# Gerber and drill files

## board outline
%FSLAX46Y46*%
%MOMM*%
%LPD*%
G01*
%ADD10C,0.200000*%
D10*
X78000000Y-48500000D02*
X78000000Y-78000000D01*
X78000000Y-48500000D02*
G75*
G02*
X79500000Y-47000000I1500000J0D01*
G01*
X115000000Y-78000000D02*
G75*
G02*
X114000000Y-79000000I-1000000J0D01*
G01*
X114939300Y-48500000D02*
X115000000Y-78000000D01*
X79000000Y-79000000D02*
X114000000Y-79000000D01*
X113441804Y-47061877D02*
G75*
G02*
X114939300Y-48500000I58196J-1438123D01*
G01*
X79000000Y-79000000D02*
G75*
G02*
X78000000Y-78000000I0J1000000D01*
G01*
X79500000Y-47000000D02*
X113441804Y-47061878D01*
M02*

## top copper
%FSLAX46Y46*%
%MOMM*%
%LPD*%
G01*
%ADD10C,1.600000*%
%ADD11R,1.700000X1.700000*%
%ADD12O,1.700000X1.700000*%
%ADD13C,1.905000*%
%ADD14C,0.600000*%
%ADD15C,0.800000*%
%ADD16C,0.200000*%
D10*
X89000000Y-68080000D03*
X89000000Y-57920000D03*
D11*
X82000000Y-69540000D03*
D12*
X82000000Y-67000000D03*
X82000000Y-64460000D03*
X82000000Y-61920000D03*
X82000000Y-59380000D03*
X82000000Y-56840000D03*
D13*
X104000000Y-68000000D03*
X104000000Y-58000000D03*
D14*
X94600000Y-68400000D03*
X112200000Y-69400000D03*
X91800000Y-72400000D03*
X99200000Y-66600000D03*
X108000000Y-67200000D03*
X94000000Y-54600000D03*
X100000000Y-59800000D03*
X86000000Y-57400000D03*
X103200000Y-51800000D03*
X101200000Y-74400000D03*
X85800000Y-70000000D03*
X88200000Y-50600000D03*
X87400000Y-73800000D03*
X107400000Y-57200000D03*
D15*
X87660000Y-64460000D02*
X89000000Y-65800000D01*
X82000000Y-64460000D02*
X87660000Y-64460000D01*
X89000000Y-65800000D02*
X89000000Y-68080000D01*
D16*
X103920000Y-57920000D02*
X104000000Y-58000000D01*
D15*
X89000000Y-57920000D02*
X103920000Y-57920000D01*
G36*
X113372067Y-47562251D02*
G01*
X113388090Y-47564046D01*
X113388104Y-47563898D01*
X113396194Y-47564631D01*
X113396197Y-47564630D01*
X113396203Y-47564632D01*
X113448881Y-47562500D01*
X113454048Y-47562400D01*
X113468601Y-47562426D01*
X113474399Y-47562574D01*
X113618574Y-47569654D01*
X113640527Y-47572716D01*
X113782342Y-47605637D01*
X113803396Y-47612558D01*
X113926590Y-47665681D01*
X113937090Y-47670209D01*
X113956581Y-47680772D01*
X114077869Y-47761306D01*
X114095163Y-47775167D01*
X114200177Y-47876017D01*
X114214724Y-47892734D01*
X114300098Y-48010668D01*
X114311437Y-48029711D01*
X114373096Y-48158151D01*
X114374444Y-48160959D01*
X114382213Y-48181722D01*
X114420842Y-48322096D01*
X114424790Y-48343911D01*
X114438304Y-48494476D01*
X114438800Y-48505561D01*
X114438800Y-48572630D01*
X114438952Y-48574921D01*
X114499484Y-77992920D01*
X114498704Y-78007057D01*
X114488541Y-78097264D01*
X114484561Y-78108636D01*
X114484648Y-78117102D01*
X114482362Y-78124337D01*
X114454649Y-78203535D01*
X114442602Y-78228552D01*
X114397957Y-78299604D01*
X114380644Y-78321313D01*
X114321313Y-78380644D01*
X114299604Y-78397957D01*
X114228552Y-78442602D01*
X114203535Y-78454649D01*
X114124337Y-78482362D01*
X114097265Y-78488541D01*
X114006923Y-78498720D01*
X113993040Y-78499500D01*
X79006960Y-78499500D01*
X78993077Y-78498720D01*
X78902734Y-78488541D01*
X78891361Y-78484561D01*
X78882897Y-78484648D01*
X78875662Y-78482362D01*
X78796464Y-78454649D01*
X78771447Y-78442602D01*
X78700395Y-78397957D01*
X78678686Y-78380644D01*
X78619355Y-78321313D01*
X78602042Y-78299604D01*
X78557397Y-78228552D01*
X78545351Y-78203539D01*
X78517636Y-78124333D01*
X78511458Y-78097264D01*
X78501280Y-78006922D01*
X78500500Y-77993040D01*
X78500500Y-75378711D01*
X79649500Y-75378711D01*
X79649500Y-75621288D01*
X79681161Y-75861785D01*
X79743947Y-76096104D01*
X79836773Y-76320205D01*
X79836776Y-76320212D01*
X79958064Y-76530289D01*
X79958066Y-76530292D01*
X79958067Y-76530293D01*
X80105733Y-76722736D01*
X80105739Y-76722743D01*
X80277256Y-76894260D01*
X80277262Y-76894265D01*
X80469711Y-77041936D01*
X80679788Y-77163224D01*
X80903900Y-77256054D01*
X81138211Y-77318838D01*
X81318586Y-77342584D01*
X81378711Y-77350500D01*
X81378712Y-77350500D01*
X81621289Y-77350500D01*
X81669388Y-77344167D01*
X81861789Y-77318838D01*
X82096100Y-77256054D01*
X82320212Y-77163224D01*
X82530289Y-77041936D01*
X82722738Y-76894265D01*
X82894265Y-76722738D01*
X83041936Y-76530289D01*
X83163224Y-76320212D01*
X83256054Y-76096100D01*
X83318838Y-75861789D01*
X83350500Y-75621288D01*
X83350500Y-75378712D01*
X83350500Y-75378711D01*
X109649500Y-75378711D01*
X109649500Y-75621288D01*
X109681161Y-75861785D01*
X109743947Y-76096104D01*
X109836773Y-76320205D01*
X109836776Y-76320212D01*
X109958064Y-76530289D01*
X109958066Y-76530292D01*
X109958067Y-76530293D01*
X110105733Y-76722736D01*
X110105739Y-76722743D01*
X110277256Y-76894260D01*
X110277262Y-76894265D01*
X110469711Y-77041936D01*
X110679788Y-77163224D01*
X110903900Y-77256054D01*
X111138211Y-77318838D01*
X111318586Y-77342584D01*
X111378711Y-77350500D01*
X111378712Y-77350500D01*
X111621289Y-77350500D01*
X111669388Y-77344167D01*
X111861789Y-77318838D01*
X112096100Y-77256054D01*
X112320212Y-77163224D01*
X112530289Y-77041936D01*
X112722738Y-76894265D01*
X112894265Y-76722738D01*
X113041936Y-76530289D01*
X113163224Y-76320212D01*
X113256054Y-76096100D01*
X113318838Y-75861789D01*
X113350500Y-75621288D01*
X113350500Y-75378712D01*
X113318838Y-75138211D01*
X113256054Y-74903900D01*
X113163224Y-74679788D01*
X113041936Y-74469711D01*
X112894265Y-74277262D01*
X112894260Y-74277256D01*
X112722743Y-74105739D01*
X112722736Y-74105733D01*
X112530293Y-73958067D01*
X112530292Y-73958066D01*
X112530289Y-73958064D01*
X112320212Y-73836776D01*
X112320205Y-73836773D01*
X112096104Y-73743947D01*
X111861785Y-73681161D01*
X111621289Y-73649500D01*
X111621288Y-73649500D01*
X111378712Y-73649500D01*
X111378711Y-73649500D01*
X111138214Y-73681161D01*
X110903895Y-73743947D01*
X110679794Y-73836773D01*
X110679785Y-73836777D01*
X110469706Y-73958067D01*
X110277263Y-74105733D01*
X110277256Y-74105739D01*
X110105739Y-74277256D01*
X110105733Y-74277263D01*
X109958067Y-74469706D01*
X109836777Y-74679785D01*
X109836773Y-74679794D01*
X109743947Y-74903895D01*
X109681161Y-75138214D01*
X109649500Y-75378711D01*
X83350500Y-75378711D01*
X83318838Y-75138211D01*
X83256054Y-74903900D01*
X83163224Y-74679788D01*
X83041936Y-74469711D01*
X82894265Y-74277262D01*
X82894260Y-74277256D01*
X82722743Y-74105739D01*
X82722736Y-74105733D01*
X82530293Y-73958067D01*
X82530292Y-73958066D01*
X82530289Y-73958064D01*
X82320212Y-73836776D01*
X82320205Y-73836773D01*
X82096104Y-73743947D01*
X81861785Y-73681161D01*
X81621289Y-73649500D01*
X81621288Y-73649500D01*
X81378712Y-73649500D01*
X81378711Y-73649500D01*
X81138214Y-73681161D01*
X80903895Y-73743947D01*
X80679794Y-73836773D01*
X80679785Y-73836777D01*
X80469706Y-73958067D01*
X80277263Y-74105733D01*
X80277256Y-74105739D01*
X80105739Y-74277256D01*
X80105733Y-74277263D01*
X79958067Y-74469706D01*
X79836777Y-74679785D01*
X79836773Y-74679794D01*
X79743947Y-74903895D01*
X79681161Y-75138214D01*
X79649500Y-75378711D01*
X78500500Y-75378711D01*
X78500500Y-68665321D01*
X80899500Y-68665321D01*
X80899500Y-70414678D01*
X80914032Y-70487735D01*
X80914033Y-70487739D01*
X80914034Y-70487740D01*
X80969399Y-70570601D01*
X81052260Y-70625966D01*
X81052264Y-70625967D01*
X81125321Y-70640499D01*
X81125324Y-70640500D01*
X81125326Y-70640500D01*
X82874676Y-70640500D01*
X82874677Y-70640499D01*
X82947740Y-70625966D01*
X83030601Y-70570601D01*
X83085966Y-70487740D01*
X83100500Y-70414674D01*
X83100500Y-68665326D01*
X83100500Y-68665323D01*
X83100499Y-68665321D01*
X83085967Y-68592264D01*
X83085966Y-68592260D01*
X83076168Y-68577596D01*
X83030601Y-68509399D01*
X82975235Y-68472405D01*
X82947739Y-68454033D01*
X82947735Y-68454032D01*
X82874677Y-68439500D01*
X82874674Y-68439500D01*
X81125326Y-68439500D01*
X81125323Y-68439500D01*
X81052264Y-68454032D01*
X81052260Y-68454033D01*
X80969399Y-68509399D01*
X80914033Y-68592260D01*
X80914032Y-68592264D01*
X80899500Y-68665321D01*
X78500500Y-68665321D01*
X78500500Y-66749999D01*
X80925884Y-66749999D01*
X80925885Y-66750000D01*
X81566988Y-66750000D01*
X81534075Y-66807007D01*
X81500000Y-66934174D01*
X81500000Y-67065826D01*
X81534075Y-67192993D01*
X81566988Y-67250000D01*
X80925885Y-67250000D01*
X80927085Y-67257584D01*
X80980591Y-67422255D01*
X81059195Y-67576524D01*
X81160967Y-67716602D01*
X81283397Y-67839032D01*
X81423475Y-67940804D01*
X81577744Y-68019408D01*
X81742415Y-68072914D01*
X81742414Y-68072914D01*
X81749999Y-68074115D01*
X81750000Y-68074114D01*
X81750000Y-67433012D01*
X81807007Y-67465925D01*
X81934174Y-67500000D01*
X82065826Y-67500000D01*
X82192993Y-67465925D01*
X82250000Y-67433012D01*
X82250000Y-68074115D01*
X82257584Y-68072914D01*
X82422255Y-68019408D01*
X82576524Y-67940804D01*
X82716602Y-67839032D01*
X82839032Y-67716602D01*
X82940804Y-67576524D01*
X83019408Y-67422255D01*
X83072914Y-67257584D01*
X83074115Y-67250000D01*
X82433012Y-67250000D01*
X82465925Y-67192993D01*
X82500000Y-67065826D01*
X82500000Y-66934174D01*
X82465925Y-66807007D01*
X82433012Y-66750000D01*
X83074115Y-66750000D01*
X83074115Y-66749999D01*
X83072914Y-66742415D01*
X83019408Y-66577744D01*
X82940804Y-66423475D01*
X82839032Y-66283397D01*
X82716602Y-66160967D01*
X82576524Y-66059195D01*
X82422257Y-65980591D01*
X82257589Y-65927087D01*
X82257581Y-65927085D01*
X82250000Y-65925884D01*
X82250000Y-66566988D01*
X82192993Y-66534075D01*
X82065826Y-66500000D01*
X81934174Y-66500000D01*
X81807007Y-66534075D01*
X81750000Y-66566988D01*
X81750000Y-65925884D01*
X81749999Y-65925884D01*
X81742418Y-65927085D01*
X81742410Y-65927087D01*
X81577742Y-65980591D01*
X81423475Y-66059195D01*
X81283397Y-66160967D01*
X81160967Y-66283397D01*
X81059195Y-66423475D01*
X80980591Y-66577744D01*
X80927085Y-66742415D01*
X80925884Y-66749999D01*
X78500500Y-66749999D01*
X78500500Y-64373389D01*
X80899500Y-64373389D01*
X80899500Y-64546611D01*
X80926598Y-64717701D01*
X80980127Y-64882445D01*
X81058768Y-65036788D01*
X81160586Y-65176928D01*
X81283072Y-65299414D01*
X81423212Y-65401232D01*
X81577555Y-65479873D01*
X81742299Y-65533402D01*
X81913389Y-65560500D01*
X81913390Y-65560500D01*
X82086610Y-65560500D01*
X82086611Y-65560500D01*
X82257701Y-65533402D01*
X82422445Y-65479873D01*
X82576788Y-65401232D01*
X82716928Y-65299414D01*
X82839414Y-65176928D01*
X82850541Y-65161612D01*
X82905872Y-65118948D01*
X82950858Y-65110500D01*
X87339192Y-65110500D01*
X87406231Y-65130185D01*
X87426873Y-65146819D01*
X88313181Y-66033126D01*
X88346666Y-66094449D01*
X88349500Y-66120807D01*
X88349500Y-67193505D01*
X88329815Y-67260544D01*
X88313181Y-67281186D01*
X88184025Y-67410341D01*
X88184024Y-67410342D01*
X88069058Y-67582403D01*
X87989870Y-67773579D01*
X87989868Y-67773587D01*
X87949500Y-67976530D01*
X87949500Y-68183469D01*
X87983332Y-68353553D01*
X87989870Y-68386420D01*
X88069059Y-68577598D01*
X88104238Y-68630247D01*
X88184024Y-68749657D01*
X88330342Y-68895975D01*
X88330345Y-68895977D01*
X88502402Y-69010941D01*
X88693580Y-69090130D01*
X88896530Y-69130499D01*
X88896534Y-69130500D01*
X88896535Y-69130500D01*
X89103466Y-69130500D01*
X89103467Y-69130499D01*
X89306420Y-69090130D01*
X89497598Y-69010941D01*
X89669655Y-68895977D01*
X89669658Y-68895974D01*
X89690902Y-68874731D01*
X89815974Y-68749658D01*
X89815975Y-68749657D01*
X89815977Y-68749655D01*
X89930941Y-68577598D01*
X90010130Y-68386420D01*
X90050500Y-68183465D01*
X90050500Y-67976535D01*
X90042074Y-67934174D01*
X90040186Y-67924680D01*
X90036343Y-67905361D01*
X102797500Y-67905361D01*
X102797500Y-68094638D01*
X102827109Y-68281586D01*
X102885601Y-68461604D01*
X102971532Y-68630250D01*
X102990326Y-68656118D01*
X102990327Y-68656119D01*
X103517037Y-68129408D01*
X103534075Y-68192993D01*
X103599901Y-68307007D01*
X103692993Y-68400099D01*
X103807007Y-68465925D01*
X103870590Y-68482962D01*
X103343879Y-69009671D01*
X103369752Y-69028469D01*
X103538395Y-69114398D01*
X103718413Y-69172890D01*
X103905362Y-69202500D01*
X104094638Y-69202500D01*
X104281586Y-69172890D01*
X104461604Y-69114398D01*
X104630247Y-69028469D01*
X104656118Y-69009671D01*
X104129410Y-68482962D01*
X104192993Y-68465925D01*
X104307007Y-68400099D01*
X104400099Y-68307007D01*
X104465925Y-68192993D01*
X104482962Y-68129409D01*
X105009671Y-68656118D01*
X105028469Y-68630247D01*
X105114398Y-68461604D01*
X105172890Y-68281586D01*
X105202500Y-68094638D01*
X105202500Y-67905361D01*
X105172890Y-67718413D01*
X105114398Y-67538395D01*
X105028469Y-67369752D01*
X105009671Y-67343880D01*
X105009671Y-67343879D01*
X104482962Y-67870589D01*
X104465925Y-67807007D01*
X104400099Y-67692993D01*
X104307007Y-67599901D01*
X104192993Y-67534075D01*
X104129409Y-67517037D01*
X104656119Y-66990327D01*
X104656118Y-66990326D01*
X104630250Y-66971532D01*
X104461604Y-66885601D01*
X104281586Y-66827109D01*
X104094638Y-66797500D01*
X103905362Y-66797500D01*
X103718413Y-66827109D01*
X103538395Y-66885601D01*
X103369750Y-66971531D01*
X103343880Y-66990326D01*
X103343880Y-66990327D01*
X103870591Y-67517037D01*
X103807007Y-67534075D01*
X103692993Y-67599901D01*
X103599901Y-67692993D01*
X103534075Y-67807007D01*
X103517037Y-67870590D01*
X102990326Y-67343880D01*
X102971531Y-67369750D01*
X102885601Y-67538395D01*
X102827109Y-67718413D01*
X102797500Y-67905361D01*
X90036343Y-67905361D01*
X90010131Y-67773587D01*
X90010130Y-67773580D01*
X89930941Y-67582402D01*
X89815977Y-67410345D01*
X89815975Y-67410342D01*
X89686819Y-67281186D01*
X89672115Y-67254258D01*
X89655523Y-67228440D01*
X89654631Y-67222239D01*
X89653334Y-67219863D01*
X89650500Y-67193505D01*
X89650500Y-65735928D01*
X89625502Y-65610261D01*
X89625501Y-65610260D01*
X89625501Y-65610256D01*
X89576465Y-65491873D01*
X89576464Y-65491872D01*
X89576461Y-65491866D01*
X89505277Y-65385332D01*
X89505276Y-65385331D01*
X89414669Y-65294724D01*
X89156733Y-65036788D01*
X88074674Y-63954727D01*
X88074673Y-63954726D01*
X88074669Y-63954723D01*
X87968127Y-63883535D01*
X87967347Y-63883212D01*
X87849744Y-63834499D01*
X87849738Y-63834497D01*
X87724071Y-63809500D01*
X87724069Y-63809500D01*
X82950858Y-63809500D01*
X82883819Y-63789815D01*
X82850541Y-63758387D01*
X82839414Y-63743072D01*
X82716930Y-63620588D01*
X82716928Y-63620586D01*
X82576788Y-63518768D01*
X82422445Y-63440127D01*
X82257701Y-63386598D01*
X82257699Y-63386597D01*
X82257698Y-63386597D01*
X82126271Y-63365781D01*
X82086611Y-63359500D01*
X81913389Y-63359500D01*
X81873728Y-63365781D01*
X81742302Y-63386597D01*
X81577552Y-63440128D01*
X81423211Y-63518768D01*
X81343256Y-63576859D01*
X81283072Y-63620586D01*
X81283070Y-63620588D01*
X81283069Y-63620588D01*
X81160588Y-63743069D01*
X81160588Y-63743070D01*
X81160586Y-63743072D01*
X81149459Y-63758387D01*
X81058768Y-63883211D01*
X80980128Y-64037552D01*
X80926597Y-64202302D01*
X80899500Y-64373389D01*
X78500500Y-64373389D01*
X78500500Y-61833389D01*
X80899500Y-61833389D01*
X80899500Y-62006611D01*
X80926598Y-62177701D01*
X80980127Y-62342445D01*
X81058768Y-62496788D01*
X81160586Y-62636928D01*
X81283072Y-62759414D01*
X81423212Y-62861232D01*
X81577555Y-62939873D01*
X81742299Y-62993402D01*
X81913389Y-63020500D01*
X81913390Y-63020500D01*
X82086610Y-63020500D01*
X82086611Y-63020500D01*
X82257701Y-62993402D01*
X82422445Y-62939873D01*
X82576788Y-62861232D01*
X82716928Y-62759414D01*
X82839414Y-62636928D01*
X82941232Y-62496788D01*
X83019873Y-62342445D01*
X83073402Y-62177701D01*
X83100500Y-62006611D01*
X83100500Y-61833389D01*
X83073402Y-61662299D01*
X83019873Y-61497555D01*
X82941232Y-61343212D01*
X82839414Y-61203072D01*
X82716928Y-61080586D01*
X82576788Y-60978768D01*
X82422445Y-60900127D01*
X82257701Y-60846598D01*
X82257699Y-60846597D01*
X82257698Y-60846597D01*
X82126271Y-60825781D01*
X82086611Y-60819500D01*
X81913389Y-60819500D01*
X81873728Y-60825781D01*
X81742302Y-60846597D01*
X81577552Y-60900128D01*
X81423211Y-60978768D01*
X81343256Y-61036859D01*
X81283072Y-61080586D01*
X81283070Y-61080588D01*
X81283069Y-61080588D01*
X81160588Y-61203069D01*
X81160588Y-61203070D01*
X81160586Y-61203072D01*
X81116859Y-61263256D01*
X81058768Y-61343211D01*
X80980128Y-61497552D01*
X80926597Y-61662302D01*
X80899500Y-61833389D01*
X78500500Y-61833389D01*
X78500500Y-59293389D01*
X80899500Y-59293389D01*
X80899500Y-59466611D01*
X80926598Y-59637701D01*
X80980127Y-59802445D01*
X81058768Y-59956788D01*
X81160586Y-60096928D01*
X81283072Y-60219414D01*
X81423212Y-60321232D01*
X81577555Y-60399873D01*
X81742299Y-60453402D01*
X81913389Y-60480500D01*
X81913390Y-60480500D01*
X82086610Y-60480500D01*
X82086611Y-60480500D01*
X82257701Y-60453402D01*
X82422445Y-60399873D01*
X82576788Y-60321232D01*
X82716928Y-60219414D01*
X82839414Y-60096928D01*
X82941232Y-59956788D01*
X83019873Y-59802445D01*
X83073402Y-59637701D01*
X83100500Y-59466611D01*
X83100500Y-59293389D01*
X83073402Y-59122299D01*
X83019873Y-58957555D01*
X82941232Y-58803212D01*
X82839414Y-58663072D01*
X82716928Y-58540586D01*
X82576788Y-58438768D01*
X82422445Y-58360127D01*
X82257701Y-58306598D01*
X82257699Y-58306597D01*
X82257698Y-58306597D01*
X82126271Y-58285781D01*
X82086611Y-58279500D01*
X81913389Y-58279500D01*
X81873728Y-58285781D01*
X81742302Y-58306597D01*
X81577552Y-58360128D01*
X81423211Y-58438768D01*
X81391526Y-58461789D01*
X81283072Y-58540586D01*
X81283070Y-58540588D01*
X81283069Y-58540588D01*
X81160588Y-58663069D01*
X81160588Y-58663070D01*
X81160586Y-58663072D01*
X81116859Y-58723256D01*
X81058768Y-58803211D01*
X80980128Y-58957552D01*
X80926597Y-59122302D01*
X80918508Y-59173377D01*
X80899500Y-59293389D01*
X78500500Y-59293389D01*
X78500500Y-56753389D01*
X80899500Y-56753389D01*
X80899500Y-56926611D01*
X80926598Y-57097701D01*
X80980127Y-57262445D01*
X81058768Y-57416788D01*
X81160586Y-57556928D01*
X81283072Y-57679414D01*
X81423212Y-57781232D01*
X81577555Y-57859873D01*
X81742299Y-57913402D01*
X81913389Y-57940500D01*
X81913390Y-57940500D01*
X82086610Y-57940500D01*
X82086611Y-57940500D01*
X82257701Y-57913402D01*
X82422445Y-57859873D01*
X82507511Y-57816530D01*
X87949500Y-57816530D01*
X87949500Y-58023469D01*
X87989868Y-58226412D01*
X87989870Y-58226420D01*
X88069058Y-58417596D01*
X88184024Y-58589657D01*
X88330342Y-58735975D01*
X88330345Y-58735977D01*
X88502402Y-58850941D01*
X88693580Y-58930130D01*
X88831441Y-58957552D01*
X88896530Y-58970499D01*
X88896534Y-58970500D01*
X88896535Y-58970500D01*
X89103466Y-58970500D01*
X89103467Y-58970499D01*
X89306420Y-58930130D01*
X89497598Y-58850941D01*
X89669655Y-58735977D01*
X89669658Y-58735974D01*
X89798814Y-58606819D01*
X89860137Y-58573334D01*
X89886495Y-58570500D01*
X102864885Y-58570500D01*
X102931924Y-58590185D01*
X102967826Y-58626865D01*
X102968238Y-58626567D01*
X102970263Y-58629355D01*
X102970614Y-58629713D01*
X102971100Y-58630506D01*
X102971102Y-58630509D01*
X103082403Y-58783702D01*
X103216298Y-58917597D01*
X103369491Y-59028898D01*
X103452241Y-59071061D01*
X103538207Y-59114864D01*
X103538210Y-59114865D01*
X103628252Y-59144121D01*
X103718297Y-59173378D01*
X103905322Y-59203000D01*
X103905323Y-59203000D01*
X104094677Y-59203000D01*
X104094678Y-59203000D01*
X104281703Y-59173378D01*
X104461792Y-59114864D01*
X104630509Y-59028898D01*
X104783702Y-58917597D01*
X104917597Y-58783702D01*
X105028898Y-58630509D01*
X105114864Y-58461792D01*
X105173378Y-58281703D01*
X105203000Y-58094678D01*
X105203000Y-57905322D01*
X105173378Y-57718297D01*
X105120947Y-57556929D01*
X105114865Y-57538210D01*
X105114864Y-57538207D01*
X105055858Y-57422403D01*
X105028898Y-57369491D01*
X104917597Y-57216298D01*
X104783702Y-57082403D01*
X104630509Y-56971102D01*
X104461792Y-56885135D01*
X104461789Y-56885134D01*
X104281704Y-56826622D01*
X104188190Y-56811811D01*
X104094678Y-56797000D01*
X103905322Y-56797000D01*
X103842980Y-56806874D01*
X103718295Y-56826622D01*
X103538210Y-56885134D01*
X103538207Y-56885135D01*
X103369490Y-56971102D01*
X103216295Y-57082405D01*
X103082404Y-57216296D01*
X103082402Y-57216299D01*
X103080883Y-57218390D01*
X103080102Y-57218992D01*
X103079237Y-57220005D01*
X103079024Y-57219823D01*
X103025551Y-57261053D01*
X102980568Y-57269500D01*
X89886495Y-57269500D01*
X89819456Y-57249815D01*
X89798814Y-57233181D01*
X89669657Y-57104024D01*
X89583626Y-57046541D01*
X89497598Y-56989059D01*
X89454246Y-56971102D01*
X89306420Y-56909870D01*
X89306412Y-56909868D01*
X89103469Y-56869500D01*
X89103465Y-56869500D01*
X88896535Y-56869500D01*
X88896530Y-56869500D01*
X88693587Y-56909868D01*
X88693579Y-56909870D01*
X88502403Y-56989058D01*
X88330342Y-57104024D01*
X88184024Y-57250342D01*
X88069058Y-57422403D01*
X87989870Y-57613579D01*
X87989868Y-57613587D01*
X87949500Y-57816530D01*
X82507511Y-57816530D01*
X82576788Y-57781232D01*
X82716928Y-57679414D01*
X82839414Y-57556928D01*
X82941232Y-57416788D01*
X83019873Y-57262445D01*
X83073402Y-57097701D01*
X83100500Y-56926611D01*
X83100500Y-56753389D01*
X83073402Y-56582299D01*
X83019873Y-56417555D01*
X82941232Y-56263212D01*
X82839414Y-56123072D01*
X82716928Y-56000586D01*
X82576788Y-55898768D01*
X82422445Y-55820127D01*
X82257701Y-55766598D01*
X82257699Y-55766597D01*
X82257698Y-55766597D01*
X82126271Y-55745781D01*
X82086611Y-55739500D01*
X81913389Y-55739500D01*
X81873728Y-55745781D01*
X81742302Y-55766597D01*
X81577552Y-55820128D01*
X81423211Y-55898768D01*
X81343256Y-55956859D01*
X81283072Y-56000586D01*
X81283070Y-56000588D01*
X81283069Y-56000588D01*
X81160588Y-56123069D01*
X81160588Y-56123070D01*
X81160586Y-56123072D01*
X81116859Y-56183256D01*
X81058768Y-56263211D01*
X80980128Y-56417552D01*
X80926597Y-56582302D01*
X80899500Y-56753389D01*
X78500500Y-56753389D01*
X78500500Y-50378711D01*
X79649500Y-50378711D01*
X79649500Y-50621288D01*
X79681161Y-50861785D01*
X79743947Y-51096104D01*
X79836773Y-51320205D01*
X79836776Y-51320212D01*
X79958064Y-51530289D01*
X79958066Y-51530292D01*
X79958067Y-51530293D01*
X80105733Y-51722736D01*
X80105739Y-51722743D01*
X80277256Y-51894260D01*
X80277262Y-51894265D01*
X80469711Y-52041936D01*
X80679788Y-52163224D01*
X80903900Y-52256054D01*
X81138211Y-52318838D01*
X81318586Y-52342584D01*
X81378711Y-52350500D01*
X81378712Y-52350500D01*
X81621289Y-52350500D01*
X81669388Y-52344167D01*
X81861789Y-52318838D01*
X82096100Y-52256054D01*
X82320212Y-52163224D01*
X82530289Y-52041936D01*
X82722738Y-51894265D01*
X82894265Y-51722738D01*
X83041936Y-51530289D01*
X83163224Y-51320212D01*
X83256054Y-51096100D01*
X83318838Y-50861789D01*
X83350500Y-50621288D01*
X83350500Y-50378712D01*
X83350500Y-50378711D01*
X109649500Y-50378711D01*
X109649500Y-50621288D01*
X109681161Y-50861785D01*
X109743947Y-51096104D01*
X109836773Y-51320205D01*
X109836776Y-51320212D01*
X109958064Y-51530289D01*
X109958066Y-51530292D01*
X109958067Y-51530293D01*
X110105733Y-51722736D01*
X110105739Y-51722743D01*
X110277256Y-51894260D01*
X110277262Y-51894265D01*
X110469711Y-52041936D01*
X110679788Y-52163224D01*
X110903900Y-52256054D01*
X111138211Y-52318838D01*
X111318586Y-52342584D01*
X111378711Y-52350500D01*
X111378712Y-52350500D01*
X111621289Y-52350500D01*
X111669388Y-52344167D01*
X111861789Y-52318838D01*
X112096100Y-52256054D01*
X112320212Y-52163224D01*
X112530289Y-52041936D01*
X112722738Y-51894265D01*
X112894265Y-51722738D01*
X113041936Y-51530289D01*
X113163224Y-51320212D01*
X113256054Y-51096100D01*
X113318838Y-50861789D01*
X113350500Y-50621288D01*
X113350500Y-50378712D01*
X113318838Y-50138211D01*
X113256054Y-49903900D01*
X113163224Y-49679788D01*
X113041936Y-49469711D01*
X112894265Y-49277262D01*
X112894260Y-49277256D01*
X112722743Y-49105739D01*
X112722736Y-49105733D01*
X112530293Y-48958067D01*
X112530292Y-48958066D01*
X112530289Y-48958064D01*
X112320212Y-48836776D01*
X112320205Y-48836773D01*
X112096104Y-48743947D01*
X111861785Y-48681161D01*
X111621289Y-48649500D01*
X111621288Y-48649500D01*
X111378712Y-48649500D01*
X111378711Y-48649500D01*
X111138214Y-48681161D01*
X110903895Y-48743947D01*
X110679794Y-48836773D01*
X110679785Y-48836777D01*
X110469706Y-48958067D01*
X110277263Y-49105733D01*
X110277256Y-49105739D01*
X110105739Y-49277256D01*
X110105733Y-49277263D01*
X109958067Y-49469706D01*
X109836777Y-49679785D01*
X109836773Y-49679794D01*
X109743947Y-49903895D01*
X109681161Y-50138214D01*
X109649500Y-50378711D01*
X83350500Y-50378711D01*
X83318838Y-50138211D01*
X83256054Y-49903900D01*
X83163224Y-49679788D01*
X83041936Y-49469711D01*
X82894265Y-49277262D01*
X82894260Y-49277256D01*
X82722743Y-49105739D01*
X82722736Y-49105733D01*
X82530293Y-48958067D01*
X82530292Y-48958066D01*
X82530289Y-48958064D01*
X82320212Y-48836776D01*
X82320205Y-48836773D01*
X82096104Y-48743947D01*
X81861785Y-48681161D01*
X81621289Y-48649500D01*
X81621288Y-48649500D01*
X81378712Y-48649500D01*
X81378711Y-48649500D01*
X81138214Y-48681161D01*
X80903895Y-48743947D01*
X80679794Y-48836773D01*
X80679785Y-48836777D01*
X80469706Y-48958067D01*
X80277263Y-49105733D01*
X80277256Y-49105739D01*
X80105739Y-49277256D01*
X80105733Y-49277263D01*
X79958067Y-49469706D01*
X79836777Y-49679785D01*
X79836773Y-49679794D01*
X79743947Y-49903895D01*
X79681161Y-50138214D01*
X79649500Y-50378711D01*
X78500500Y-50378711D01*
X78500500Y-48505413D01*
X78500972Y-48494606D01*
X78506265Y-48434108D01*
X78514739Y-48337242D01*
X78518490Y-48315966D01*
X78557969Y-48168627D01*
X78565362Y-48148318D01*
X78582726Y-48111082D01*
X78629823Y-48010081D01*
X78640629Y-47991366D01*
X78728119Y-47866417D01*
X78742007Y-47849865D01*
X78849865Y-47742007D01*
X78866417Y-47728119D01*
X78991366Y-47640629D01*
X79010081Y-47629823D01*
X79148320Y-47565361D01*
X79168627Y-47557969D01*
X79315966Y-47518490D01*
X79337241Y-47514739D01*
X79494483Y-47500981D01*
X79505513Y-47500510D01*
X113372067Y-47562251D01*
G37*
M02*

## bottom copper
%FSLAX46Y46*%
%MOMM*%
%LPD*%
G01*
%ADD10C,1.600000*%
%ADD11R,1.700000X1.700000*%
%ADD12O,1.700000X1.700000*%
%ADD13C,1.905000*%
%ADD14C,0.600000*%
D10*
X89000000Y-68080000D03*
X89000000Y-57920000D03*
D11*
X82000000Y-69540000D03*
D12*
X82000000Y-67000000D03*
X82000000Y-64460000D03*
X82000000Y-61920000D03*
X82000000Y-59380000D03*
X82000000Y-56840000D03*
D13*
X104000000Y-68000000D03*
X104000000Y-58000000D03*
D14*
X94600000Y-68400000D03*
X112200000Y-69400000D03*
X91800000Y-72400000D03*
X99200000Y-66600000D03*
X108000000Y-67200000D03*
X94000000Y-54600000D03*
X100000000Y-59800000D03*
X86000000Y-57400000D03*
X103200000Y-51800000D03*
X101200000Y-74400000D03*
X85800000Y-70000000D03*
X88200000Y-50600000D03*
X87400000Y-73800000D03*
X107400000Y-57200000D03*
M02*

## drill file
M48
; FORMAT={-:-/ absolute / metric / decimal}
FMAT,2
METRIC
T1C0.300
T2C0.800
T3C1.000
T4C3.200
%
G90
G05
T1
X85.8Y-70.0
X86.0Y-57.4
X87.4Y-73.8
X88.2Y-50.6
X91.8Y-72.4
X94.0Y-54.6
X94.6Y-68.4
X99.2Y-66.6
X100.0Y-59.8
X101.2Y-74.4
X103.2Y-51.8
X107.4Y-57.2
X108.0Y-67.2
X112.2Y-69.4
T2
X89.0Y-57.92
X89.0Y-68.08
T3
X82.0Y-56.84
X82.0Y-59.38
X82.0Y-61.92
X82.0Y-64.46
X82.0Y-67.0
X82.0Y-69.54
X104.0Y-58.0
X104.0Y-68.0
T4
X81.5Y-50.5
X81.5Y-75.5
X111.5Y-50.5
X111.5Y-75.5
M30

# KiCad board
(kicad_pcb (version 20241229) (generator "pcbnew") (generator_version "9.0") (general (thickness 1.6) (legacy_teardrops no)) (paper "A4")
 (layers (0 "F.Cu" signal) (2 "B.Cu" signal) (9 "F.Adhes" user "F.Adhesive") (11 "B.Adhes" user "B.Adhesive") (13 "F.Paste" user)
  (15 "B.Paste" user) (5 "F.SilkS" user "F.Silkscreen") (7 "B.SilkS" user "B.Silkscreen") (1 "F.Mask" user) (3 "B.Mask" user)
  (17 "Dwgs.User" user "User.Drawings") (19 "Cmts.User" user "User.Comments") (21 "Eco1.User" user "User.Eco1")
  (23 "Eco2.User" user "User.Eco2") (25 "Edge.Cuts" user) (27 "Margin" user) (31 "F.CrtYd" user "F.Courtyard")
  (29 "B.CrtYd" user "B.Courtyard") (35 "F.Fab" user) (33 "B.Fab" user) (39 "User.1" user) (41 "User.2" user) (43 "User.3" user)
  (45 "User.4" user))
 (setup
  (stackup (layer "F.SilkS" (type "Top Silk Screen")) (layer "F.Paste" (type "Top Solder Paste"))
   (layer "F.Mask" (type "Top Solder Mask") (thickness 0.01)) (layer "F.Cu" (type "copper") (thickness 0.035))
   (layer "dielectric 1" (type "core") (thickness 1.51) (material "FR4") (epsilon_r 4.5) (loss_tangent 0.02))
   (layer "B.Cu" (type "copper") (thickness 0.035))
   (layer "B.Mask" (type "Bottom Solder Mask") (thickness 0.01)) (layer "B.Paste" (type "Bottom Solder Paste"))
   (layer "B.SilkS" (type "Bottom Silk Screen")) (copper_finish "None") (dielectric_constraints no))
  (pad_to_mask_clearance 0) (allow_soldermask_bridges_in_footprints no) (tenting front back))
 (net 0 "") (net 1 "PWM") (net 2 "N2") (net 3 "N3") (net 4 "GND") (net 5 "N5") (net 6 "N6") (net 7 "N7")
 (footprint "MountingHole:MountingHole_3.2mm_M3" (layer "F.Cu") (at 111.5 50.5)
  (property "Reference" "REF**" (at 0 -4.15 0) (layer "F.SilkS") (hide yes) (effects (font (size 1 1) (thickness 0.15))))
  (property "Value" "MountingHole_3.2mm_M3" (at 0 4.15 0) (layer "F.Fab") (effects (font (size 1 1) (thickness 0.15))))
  (pad "" np_thru_hole circle (at 0 0) (size 3.2 3.2) (drill 3.2) (layers "*.Cu" "*.Mask")))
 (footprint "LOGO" (layer "F.Cu") (at 96 73)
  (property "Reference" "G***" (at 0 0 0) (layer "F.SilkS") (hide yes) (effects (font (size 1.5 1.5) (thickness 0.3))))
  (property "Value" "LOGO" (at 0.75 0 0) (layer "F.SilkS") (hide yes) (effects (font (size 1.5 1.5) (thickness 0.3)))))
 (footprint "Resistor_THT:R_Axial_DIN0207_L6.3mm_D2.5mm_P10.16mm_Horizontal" (layer "F.Cu") (at 89 68.08 90)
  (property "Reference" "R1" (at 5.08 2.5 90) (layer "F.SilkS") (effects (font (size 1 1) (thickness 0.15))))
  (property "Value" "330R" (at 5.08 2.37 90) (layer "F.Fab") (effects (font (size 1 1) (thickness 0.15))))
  (pad "1" thru_hole circle (at 0 0 90) (size 1.6 1.6) (drill 0.8) (layers "*.Cu" "*.Mask") (remove_unused_layers no) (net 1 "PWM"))
  (pad "2" thru_hole circle (at 10.16 0 90) (size 1.6 1.6) (drill 0.8) (layers "*.Cu" "*.Mask") (remove_unused_layers no) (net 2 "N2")))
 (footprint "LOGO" (layer "F.Cu") (at 98.5 63)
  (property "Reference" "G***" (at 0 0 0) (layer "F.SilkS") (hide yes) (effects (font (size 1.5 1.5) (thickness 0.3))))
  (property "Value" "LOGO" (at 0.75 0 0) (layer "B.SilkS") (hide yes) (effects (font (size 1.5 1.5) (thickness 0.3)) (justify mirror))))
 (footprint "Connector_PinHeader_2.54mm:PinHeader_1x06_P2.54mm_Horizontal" (layer "F.Cu") (at 82 69.54 180)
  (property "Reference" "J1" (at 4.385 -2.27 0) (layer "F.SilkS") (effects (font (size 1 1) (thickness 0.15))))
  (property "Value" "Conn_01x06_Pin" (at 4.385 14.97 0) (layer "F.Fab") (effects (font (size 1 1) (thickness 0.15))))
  (pad "1" thru_hole rect (at 0 0 180) (size 1.7 1.7) (drill 1) (layers "*.Cu" "*.Mask") (remove_unused_layers no) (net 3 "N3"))
  (pad "2" thru_hole oval (at 0 2.54 180) (size 1.7 1.7) (drill 1) (layers "*.Cu" "*.Mask") (remove_unused_layers no) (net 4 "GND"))
  (pad "3" thru_hole oval (at 0 5.08 180) (size 1.7 1.7) (drill 1) (layers "*.Cu" "*.Mask") (remove_unused_layers no) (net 1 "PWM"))
  (pad "4" thru_hole oval (at 0 7.62 180) (size 1.7 1.7) (drill 1) (layers "*.Cu" "*.Mask") (remove_unused_layers no) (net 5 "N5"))
  (pad "5" thru_hole oval (at 0 10.16 180) (size 1.7 1.7) (drill 1) (layers "*.Cu" "*.Mask") (remove_unused_layers no) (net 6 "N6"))
  (pad "6" thru_hole oval (at 0 12.7 180) (size 1.7 1.7) (drill 1) (layers "*.Cu" "*.Mask") (remove_unused_layers no) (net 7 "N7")))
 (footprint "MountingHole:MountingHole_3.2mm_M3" (layer "F.Cu") (at 81.5 50.5)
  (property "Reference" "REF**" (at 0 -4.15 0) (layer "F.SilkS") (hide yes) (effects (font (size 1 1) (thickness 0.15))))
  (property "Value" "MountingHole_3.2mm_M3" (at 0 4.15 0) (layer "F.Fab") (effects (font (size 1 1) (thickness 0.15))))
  (pad "" np_thru_hole circle (at 0 0) (size 3.2 3.2) (drill 3.2) (layers "*.Cu" "*.Mask")))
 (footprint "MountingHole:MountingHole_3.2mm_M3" (layer "F.Cu") (at 111.5 75.5)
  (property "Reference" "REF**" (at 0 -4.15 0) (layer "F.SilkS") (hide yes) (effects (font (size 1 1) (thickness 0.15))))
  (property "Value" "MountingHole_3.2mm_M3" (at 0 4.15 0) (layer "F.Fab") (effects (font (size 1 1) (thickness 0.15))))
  (pad "" np_thru_hole circle (at 0 0) (size 3.2 3.2) (drill 3.2) (layers "*.Cu" "*.Mask")))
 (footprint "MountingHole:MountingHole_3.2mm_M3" (layer "F.Cu") (at 81.5 75.5)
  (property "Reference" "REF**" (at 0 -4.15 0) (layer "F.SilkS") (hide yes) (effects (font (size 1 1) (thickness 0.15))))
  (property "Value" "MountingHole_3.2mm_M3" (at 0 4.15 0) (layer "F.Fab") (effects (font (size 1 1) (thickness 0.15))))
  (pad "" np_thru_hole circle (at 0 0) (size 3.2 3.2) (drill 3.2) (layers "*.Cu" "*.Mask")))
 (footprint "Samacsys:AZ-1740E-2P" (layer "F.Cu") (at 104 63 -90)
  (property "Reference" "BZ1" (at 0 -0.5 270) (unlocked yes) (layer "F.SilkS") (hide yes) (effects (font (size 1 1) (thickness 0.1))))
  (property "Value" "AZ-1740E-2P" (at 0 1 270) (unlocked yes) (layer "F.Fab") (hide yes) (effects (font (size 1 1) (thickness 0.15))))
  (pad "1" thru_hole circle (at 5 0 270) (size 1.905 1.905) (drill 1) (layers "*.Cu" "*.Mask") (remove_unused_layers no) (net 4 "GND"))
  (pad "2" thru_hole circle (at -5 0 270) (size 1.905 1.905) (drill 1) (layers "*.Cu" "*.Mask") (remove_unused_layers no) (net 2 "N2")))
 (gr_line (start 78 48.5) (end 78 78) (stroke (width 0.2) (type solid)) (layer "Edge.Cuts"))
 (gr_arc (start 78 48.5) (mid 78.43934 47.43934) (end 79.5 47) (stroke (width 0.2) (type solid)) (layer "Edge.Cuts"))
 (gr_arc (start 115 78) (mid 114.707107 78.707107) (end 114 79) (stroke (width 0.2) (type solid)) (layer "Edge.Cuts"))
 (gr_line (start 114.9393 48.5) (end 115 78) (stroke (width 0.2) (type solid)) (layer "Edge.Cuts"))
 (gr_line (start 79 79) (end 114 79) (stroke (width 0.2) (type solid)) (layer "Edge.Cuts"))
 (gr_arc (start 113.441804 47.061877) (mid 114.496951 47.46189) (end 114.9393 48.5) (stroke (width 0.2) (type solid)) (layer "Edge.Cuts"))
 (gr_arc (start 79 79) (mid 78.292893 78.707107) (end 78 78) (stroke (width 0.2) (type solid)) (layer "Edge.Cuts"))
 (gr_line (start 79.5 47) (end 113.441804 47.061878) (stroke (width 0.2) (type solid)) (layer "Edge.Cuts"))
 (via (at 94.6 68.4) (size 0.6) (drill 0.3) (layers "F.Cu" "B.Cu") (free yes) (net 4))
 (via (at 112.2 69.4) (size 0.6) (drill 0.3) (layers "F.Cu" "B.Cu") (free yes) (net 4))
 (via (at 91.8 72.4) (size 0.6) (drill 0.3) (layers "F.Cu" "B.Cu") (free yes) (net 4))
 (via (at 99.2 66.6) (size 0.6) (drill 0.3) (layers "F.Cu" "B.Cu") (free yes) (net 4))
 (via (at 108 67.2) (size 0.6) (drill 0.3) (layers "F.Cu" "B.Cu") (free yes) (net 4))
 (via (at 94 54.6) (size 0.6) (drill 0.3) (layers "F.Cu" "B.Cu") (free yes) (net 4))
 (via (at 100 59.8) (size 0.6) (drill 0.3) (layers "F.Cu" "B.Cu") (free yes) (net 4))
 (via (at 86 57.4) (size 0.6) (drill 0.3) (layers "F.Cu" "B.Cu") (free yes) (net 4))
 (via (at 103.2 51.8) (size 0.6) (drill 0.3) (layers "F.Cu" "B.Cu") (free yes) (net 4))
 (via (at 101.2 74.4) (size 0.6) (drill 0.3) (layers "F.Cu" "B.Cu") (free yes) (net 4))
 (via (at 85.8 70) (size 0.6) (drill 0.3) (layers "F.Cu" "B.Cu") (free yes) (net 4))
 (via (at 88.2 50.6) (size 0.6) (drill 0.3) (layers "F.Cu" "B.Cu") (free yes) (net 4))
 (via (at 87.4 73.8) (size 0.6) (drill 0.3) (layers "F.Cu" "B.Cu") (free yes) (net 4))
 (via (at 107.4 57.2) (size 0.6) (drill 0.3) (layers "F.Cu" "B.Cu") (free yes) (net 4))
 (segment (start 87.66 64.46) (end 89 65.8) (width 0.8) (layer "F.Cu") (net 1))
 (segment (start 82 64.46) (end 87.66 64.46) (width 0.8) (layer "F.Cu") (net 1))
 (segment (start 89 65.8) (end 89 68.08) (width 0.8) (layer "F.Cu") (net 1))
 (segment (start 103.92 57.92) (end 104 58) (width 0.2) (layer "F.Cu") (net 2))
 (segment (start 89 57.92) (end 103.92 57.92) (width 0.8) (layer "F.Cu") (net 2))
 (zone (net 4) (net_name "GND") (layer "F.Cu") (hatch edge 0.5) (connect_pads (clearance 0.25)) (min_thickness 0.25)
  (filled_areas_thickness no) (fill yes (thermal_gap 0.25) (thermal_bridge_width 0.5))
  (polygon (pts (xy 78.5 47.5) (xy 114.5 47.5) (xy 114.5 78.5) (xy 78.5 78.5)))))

